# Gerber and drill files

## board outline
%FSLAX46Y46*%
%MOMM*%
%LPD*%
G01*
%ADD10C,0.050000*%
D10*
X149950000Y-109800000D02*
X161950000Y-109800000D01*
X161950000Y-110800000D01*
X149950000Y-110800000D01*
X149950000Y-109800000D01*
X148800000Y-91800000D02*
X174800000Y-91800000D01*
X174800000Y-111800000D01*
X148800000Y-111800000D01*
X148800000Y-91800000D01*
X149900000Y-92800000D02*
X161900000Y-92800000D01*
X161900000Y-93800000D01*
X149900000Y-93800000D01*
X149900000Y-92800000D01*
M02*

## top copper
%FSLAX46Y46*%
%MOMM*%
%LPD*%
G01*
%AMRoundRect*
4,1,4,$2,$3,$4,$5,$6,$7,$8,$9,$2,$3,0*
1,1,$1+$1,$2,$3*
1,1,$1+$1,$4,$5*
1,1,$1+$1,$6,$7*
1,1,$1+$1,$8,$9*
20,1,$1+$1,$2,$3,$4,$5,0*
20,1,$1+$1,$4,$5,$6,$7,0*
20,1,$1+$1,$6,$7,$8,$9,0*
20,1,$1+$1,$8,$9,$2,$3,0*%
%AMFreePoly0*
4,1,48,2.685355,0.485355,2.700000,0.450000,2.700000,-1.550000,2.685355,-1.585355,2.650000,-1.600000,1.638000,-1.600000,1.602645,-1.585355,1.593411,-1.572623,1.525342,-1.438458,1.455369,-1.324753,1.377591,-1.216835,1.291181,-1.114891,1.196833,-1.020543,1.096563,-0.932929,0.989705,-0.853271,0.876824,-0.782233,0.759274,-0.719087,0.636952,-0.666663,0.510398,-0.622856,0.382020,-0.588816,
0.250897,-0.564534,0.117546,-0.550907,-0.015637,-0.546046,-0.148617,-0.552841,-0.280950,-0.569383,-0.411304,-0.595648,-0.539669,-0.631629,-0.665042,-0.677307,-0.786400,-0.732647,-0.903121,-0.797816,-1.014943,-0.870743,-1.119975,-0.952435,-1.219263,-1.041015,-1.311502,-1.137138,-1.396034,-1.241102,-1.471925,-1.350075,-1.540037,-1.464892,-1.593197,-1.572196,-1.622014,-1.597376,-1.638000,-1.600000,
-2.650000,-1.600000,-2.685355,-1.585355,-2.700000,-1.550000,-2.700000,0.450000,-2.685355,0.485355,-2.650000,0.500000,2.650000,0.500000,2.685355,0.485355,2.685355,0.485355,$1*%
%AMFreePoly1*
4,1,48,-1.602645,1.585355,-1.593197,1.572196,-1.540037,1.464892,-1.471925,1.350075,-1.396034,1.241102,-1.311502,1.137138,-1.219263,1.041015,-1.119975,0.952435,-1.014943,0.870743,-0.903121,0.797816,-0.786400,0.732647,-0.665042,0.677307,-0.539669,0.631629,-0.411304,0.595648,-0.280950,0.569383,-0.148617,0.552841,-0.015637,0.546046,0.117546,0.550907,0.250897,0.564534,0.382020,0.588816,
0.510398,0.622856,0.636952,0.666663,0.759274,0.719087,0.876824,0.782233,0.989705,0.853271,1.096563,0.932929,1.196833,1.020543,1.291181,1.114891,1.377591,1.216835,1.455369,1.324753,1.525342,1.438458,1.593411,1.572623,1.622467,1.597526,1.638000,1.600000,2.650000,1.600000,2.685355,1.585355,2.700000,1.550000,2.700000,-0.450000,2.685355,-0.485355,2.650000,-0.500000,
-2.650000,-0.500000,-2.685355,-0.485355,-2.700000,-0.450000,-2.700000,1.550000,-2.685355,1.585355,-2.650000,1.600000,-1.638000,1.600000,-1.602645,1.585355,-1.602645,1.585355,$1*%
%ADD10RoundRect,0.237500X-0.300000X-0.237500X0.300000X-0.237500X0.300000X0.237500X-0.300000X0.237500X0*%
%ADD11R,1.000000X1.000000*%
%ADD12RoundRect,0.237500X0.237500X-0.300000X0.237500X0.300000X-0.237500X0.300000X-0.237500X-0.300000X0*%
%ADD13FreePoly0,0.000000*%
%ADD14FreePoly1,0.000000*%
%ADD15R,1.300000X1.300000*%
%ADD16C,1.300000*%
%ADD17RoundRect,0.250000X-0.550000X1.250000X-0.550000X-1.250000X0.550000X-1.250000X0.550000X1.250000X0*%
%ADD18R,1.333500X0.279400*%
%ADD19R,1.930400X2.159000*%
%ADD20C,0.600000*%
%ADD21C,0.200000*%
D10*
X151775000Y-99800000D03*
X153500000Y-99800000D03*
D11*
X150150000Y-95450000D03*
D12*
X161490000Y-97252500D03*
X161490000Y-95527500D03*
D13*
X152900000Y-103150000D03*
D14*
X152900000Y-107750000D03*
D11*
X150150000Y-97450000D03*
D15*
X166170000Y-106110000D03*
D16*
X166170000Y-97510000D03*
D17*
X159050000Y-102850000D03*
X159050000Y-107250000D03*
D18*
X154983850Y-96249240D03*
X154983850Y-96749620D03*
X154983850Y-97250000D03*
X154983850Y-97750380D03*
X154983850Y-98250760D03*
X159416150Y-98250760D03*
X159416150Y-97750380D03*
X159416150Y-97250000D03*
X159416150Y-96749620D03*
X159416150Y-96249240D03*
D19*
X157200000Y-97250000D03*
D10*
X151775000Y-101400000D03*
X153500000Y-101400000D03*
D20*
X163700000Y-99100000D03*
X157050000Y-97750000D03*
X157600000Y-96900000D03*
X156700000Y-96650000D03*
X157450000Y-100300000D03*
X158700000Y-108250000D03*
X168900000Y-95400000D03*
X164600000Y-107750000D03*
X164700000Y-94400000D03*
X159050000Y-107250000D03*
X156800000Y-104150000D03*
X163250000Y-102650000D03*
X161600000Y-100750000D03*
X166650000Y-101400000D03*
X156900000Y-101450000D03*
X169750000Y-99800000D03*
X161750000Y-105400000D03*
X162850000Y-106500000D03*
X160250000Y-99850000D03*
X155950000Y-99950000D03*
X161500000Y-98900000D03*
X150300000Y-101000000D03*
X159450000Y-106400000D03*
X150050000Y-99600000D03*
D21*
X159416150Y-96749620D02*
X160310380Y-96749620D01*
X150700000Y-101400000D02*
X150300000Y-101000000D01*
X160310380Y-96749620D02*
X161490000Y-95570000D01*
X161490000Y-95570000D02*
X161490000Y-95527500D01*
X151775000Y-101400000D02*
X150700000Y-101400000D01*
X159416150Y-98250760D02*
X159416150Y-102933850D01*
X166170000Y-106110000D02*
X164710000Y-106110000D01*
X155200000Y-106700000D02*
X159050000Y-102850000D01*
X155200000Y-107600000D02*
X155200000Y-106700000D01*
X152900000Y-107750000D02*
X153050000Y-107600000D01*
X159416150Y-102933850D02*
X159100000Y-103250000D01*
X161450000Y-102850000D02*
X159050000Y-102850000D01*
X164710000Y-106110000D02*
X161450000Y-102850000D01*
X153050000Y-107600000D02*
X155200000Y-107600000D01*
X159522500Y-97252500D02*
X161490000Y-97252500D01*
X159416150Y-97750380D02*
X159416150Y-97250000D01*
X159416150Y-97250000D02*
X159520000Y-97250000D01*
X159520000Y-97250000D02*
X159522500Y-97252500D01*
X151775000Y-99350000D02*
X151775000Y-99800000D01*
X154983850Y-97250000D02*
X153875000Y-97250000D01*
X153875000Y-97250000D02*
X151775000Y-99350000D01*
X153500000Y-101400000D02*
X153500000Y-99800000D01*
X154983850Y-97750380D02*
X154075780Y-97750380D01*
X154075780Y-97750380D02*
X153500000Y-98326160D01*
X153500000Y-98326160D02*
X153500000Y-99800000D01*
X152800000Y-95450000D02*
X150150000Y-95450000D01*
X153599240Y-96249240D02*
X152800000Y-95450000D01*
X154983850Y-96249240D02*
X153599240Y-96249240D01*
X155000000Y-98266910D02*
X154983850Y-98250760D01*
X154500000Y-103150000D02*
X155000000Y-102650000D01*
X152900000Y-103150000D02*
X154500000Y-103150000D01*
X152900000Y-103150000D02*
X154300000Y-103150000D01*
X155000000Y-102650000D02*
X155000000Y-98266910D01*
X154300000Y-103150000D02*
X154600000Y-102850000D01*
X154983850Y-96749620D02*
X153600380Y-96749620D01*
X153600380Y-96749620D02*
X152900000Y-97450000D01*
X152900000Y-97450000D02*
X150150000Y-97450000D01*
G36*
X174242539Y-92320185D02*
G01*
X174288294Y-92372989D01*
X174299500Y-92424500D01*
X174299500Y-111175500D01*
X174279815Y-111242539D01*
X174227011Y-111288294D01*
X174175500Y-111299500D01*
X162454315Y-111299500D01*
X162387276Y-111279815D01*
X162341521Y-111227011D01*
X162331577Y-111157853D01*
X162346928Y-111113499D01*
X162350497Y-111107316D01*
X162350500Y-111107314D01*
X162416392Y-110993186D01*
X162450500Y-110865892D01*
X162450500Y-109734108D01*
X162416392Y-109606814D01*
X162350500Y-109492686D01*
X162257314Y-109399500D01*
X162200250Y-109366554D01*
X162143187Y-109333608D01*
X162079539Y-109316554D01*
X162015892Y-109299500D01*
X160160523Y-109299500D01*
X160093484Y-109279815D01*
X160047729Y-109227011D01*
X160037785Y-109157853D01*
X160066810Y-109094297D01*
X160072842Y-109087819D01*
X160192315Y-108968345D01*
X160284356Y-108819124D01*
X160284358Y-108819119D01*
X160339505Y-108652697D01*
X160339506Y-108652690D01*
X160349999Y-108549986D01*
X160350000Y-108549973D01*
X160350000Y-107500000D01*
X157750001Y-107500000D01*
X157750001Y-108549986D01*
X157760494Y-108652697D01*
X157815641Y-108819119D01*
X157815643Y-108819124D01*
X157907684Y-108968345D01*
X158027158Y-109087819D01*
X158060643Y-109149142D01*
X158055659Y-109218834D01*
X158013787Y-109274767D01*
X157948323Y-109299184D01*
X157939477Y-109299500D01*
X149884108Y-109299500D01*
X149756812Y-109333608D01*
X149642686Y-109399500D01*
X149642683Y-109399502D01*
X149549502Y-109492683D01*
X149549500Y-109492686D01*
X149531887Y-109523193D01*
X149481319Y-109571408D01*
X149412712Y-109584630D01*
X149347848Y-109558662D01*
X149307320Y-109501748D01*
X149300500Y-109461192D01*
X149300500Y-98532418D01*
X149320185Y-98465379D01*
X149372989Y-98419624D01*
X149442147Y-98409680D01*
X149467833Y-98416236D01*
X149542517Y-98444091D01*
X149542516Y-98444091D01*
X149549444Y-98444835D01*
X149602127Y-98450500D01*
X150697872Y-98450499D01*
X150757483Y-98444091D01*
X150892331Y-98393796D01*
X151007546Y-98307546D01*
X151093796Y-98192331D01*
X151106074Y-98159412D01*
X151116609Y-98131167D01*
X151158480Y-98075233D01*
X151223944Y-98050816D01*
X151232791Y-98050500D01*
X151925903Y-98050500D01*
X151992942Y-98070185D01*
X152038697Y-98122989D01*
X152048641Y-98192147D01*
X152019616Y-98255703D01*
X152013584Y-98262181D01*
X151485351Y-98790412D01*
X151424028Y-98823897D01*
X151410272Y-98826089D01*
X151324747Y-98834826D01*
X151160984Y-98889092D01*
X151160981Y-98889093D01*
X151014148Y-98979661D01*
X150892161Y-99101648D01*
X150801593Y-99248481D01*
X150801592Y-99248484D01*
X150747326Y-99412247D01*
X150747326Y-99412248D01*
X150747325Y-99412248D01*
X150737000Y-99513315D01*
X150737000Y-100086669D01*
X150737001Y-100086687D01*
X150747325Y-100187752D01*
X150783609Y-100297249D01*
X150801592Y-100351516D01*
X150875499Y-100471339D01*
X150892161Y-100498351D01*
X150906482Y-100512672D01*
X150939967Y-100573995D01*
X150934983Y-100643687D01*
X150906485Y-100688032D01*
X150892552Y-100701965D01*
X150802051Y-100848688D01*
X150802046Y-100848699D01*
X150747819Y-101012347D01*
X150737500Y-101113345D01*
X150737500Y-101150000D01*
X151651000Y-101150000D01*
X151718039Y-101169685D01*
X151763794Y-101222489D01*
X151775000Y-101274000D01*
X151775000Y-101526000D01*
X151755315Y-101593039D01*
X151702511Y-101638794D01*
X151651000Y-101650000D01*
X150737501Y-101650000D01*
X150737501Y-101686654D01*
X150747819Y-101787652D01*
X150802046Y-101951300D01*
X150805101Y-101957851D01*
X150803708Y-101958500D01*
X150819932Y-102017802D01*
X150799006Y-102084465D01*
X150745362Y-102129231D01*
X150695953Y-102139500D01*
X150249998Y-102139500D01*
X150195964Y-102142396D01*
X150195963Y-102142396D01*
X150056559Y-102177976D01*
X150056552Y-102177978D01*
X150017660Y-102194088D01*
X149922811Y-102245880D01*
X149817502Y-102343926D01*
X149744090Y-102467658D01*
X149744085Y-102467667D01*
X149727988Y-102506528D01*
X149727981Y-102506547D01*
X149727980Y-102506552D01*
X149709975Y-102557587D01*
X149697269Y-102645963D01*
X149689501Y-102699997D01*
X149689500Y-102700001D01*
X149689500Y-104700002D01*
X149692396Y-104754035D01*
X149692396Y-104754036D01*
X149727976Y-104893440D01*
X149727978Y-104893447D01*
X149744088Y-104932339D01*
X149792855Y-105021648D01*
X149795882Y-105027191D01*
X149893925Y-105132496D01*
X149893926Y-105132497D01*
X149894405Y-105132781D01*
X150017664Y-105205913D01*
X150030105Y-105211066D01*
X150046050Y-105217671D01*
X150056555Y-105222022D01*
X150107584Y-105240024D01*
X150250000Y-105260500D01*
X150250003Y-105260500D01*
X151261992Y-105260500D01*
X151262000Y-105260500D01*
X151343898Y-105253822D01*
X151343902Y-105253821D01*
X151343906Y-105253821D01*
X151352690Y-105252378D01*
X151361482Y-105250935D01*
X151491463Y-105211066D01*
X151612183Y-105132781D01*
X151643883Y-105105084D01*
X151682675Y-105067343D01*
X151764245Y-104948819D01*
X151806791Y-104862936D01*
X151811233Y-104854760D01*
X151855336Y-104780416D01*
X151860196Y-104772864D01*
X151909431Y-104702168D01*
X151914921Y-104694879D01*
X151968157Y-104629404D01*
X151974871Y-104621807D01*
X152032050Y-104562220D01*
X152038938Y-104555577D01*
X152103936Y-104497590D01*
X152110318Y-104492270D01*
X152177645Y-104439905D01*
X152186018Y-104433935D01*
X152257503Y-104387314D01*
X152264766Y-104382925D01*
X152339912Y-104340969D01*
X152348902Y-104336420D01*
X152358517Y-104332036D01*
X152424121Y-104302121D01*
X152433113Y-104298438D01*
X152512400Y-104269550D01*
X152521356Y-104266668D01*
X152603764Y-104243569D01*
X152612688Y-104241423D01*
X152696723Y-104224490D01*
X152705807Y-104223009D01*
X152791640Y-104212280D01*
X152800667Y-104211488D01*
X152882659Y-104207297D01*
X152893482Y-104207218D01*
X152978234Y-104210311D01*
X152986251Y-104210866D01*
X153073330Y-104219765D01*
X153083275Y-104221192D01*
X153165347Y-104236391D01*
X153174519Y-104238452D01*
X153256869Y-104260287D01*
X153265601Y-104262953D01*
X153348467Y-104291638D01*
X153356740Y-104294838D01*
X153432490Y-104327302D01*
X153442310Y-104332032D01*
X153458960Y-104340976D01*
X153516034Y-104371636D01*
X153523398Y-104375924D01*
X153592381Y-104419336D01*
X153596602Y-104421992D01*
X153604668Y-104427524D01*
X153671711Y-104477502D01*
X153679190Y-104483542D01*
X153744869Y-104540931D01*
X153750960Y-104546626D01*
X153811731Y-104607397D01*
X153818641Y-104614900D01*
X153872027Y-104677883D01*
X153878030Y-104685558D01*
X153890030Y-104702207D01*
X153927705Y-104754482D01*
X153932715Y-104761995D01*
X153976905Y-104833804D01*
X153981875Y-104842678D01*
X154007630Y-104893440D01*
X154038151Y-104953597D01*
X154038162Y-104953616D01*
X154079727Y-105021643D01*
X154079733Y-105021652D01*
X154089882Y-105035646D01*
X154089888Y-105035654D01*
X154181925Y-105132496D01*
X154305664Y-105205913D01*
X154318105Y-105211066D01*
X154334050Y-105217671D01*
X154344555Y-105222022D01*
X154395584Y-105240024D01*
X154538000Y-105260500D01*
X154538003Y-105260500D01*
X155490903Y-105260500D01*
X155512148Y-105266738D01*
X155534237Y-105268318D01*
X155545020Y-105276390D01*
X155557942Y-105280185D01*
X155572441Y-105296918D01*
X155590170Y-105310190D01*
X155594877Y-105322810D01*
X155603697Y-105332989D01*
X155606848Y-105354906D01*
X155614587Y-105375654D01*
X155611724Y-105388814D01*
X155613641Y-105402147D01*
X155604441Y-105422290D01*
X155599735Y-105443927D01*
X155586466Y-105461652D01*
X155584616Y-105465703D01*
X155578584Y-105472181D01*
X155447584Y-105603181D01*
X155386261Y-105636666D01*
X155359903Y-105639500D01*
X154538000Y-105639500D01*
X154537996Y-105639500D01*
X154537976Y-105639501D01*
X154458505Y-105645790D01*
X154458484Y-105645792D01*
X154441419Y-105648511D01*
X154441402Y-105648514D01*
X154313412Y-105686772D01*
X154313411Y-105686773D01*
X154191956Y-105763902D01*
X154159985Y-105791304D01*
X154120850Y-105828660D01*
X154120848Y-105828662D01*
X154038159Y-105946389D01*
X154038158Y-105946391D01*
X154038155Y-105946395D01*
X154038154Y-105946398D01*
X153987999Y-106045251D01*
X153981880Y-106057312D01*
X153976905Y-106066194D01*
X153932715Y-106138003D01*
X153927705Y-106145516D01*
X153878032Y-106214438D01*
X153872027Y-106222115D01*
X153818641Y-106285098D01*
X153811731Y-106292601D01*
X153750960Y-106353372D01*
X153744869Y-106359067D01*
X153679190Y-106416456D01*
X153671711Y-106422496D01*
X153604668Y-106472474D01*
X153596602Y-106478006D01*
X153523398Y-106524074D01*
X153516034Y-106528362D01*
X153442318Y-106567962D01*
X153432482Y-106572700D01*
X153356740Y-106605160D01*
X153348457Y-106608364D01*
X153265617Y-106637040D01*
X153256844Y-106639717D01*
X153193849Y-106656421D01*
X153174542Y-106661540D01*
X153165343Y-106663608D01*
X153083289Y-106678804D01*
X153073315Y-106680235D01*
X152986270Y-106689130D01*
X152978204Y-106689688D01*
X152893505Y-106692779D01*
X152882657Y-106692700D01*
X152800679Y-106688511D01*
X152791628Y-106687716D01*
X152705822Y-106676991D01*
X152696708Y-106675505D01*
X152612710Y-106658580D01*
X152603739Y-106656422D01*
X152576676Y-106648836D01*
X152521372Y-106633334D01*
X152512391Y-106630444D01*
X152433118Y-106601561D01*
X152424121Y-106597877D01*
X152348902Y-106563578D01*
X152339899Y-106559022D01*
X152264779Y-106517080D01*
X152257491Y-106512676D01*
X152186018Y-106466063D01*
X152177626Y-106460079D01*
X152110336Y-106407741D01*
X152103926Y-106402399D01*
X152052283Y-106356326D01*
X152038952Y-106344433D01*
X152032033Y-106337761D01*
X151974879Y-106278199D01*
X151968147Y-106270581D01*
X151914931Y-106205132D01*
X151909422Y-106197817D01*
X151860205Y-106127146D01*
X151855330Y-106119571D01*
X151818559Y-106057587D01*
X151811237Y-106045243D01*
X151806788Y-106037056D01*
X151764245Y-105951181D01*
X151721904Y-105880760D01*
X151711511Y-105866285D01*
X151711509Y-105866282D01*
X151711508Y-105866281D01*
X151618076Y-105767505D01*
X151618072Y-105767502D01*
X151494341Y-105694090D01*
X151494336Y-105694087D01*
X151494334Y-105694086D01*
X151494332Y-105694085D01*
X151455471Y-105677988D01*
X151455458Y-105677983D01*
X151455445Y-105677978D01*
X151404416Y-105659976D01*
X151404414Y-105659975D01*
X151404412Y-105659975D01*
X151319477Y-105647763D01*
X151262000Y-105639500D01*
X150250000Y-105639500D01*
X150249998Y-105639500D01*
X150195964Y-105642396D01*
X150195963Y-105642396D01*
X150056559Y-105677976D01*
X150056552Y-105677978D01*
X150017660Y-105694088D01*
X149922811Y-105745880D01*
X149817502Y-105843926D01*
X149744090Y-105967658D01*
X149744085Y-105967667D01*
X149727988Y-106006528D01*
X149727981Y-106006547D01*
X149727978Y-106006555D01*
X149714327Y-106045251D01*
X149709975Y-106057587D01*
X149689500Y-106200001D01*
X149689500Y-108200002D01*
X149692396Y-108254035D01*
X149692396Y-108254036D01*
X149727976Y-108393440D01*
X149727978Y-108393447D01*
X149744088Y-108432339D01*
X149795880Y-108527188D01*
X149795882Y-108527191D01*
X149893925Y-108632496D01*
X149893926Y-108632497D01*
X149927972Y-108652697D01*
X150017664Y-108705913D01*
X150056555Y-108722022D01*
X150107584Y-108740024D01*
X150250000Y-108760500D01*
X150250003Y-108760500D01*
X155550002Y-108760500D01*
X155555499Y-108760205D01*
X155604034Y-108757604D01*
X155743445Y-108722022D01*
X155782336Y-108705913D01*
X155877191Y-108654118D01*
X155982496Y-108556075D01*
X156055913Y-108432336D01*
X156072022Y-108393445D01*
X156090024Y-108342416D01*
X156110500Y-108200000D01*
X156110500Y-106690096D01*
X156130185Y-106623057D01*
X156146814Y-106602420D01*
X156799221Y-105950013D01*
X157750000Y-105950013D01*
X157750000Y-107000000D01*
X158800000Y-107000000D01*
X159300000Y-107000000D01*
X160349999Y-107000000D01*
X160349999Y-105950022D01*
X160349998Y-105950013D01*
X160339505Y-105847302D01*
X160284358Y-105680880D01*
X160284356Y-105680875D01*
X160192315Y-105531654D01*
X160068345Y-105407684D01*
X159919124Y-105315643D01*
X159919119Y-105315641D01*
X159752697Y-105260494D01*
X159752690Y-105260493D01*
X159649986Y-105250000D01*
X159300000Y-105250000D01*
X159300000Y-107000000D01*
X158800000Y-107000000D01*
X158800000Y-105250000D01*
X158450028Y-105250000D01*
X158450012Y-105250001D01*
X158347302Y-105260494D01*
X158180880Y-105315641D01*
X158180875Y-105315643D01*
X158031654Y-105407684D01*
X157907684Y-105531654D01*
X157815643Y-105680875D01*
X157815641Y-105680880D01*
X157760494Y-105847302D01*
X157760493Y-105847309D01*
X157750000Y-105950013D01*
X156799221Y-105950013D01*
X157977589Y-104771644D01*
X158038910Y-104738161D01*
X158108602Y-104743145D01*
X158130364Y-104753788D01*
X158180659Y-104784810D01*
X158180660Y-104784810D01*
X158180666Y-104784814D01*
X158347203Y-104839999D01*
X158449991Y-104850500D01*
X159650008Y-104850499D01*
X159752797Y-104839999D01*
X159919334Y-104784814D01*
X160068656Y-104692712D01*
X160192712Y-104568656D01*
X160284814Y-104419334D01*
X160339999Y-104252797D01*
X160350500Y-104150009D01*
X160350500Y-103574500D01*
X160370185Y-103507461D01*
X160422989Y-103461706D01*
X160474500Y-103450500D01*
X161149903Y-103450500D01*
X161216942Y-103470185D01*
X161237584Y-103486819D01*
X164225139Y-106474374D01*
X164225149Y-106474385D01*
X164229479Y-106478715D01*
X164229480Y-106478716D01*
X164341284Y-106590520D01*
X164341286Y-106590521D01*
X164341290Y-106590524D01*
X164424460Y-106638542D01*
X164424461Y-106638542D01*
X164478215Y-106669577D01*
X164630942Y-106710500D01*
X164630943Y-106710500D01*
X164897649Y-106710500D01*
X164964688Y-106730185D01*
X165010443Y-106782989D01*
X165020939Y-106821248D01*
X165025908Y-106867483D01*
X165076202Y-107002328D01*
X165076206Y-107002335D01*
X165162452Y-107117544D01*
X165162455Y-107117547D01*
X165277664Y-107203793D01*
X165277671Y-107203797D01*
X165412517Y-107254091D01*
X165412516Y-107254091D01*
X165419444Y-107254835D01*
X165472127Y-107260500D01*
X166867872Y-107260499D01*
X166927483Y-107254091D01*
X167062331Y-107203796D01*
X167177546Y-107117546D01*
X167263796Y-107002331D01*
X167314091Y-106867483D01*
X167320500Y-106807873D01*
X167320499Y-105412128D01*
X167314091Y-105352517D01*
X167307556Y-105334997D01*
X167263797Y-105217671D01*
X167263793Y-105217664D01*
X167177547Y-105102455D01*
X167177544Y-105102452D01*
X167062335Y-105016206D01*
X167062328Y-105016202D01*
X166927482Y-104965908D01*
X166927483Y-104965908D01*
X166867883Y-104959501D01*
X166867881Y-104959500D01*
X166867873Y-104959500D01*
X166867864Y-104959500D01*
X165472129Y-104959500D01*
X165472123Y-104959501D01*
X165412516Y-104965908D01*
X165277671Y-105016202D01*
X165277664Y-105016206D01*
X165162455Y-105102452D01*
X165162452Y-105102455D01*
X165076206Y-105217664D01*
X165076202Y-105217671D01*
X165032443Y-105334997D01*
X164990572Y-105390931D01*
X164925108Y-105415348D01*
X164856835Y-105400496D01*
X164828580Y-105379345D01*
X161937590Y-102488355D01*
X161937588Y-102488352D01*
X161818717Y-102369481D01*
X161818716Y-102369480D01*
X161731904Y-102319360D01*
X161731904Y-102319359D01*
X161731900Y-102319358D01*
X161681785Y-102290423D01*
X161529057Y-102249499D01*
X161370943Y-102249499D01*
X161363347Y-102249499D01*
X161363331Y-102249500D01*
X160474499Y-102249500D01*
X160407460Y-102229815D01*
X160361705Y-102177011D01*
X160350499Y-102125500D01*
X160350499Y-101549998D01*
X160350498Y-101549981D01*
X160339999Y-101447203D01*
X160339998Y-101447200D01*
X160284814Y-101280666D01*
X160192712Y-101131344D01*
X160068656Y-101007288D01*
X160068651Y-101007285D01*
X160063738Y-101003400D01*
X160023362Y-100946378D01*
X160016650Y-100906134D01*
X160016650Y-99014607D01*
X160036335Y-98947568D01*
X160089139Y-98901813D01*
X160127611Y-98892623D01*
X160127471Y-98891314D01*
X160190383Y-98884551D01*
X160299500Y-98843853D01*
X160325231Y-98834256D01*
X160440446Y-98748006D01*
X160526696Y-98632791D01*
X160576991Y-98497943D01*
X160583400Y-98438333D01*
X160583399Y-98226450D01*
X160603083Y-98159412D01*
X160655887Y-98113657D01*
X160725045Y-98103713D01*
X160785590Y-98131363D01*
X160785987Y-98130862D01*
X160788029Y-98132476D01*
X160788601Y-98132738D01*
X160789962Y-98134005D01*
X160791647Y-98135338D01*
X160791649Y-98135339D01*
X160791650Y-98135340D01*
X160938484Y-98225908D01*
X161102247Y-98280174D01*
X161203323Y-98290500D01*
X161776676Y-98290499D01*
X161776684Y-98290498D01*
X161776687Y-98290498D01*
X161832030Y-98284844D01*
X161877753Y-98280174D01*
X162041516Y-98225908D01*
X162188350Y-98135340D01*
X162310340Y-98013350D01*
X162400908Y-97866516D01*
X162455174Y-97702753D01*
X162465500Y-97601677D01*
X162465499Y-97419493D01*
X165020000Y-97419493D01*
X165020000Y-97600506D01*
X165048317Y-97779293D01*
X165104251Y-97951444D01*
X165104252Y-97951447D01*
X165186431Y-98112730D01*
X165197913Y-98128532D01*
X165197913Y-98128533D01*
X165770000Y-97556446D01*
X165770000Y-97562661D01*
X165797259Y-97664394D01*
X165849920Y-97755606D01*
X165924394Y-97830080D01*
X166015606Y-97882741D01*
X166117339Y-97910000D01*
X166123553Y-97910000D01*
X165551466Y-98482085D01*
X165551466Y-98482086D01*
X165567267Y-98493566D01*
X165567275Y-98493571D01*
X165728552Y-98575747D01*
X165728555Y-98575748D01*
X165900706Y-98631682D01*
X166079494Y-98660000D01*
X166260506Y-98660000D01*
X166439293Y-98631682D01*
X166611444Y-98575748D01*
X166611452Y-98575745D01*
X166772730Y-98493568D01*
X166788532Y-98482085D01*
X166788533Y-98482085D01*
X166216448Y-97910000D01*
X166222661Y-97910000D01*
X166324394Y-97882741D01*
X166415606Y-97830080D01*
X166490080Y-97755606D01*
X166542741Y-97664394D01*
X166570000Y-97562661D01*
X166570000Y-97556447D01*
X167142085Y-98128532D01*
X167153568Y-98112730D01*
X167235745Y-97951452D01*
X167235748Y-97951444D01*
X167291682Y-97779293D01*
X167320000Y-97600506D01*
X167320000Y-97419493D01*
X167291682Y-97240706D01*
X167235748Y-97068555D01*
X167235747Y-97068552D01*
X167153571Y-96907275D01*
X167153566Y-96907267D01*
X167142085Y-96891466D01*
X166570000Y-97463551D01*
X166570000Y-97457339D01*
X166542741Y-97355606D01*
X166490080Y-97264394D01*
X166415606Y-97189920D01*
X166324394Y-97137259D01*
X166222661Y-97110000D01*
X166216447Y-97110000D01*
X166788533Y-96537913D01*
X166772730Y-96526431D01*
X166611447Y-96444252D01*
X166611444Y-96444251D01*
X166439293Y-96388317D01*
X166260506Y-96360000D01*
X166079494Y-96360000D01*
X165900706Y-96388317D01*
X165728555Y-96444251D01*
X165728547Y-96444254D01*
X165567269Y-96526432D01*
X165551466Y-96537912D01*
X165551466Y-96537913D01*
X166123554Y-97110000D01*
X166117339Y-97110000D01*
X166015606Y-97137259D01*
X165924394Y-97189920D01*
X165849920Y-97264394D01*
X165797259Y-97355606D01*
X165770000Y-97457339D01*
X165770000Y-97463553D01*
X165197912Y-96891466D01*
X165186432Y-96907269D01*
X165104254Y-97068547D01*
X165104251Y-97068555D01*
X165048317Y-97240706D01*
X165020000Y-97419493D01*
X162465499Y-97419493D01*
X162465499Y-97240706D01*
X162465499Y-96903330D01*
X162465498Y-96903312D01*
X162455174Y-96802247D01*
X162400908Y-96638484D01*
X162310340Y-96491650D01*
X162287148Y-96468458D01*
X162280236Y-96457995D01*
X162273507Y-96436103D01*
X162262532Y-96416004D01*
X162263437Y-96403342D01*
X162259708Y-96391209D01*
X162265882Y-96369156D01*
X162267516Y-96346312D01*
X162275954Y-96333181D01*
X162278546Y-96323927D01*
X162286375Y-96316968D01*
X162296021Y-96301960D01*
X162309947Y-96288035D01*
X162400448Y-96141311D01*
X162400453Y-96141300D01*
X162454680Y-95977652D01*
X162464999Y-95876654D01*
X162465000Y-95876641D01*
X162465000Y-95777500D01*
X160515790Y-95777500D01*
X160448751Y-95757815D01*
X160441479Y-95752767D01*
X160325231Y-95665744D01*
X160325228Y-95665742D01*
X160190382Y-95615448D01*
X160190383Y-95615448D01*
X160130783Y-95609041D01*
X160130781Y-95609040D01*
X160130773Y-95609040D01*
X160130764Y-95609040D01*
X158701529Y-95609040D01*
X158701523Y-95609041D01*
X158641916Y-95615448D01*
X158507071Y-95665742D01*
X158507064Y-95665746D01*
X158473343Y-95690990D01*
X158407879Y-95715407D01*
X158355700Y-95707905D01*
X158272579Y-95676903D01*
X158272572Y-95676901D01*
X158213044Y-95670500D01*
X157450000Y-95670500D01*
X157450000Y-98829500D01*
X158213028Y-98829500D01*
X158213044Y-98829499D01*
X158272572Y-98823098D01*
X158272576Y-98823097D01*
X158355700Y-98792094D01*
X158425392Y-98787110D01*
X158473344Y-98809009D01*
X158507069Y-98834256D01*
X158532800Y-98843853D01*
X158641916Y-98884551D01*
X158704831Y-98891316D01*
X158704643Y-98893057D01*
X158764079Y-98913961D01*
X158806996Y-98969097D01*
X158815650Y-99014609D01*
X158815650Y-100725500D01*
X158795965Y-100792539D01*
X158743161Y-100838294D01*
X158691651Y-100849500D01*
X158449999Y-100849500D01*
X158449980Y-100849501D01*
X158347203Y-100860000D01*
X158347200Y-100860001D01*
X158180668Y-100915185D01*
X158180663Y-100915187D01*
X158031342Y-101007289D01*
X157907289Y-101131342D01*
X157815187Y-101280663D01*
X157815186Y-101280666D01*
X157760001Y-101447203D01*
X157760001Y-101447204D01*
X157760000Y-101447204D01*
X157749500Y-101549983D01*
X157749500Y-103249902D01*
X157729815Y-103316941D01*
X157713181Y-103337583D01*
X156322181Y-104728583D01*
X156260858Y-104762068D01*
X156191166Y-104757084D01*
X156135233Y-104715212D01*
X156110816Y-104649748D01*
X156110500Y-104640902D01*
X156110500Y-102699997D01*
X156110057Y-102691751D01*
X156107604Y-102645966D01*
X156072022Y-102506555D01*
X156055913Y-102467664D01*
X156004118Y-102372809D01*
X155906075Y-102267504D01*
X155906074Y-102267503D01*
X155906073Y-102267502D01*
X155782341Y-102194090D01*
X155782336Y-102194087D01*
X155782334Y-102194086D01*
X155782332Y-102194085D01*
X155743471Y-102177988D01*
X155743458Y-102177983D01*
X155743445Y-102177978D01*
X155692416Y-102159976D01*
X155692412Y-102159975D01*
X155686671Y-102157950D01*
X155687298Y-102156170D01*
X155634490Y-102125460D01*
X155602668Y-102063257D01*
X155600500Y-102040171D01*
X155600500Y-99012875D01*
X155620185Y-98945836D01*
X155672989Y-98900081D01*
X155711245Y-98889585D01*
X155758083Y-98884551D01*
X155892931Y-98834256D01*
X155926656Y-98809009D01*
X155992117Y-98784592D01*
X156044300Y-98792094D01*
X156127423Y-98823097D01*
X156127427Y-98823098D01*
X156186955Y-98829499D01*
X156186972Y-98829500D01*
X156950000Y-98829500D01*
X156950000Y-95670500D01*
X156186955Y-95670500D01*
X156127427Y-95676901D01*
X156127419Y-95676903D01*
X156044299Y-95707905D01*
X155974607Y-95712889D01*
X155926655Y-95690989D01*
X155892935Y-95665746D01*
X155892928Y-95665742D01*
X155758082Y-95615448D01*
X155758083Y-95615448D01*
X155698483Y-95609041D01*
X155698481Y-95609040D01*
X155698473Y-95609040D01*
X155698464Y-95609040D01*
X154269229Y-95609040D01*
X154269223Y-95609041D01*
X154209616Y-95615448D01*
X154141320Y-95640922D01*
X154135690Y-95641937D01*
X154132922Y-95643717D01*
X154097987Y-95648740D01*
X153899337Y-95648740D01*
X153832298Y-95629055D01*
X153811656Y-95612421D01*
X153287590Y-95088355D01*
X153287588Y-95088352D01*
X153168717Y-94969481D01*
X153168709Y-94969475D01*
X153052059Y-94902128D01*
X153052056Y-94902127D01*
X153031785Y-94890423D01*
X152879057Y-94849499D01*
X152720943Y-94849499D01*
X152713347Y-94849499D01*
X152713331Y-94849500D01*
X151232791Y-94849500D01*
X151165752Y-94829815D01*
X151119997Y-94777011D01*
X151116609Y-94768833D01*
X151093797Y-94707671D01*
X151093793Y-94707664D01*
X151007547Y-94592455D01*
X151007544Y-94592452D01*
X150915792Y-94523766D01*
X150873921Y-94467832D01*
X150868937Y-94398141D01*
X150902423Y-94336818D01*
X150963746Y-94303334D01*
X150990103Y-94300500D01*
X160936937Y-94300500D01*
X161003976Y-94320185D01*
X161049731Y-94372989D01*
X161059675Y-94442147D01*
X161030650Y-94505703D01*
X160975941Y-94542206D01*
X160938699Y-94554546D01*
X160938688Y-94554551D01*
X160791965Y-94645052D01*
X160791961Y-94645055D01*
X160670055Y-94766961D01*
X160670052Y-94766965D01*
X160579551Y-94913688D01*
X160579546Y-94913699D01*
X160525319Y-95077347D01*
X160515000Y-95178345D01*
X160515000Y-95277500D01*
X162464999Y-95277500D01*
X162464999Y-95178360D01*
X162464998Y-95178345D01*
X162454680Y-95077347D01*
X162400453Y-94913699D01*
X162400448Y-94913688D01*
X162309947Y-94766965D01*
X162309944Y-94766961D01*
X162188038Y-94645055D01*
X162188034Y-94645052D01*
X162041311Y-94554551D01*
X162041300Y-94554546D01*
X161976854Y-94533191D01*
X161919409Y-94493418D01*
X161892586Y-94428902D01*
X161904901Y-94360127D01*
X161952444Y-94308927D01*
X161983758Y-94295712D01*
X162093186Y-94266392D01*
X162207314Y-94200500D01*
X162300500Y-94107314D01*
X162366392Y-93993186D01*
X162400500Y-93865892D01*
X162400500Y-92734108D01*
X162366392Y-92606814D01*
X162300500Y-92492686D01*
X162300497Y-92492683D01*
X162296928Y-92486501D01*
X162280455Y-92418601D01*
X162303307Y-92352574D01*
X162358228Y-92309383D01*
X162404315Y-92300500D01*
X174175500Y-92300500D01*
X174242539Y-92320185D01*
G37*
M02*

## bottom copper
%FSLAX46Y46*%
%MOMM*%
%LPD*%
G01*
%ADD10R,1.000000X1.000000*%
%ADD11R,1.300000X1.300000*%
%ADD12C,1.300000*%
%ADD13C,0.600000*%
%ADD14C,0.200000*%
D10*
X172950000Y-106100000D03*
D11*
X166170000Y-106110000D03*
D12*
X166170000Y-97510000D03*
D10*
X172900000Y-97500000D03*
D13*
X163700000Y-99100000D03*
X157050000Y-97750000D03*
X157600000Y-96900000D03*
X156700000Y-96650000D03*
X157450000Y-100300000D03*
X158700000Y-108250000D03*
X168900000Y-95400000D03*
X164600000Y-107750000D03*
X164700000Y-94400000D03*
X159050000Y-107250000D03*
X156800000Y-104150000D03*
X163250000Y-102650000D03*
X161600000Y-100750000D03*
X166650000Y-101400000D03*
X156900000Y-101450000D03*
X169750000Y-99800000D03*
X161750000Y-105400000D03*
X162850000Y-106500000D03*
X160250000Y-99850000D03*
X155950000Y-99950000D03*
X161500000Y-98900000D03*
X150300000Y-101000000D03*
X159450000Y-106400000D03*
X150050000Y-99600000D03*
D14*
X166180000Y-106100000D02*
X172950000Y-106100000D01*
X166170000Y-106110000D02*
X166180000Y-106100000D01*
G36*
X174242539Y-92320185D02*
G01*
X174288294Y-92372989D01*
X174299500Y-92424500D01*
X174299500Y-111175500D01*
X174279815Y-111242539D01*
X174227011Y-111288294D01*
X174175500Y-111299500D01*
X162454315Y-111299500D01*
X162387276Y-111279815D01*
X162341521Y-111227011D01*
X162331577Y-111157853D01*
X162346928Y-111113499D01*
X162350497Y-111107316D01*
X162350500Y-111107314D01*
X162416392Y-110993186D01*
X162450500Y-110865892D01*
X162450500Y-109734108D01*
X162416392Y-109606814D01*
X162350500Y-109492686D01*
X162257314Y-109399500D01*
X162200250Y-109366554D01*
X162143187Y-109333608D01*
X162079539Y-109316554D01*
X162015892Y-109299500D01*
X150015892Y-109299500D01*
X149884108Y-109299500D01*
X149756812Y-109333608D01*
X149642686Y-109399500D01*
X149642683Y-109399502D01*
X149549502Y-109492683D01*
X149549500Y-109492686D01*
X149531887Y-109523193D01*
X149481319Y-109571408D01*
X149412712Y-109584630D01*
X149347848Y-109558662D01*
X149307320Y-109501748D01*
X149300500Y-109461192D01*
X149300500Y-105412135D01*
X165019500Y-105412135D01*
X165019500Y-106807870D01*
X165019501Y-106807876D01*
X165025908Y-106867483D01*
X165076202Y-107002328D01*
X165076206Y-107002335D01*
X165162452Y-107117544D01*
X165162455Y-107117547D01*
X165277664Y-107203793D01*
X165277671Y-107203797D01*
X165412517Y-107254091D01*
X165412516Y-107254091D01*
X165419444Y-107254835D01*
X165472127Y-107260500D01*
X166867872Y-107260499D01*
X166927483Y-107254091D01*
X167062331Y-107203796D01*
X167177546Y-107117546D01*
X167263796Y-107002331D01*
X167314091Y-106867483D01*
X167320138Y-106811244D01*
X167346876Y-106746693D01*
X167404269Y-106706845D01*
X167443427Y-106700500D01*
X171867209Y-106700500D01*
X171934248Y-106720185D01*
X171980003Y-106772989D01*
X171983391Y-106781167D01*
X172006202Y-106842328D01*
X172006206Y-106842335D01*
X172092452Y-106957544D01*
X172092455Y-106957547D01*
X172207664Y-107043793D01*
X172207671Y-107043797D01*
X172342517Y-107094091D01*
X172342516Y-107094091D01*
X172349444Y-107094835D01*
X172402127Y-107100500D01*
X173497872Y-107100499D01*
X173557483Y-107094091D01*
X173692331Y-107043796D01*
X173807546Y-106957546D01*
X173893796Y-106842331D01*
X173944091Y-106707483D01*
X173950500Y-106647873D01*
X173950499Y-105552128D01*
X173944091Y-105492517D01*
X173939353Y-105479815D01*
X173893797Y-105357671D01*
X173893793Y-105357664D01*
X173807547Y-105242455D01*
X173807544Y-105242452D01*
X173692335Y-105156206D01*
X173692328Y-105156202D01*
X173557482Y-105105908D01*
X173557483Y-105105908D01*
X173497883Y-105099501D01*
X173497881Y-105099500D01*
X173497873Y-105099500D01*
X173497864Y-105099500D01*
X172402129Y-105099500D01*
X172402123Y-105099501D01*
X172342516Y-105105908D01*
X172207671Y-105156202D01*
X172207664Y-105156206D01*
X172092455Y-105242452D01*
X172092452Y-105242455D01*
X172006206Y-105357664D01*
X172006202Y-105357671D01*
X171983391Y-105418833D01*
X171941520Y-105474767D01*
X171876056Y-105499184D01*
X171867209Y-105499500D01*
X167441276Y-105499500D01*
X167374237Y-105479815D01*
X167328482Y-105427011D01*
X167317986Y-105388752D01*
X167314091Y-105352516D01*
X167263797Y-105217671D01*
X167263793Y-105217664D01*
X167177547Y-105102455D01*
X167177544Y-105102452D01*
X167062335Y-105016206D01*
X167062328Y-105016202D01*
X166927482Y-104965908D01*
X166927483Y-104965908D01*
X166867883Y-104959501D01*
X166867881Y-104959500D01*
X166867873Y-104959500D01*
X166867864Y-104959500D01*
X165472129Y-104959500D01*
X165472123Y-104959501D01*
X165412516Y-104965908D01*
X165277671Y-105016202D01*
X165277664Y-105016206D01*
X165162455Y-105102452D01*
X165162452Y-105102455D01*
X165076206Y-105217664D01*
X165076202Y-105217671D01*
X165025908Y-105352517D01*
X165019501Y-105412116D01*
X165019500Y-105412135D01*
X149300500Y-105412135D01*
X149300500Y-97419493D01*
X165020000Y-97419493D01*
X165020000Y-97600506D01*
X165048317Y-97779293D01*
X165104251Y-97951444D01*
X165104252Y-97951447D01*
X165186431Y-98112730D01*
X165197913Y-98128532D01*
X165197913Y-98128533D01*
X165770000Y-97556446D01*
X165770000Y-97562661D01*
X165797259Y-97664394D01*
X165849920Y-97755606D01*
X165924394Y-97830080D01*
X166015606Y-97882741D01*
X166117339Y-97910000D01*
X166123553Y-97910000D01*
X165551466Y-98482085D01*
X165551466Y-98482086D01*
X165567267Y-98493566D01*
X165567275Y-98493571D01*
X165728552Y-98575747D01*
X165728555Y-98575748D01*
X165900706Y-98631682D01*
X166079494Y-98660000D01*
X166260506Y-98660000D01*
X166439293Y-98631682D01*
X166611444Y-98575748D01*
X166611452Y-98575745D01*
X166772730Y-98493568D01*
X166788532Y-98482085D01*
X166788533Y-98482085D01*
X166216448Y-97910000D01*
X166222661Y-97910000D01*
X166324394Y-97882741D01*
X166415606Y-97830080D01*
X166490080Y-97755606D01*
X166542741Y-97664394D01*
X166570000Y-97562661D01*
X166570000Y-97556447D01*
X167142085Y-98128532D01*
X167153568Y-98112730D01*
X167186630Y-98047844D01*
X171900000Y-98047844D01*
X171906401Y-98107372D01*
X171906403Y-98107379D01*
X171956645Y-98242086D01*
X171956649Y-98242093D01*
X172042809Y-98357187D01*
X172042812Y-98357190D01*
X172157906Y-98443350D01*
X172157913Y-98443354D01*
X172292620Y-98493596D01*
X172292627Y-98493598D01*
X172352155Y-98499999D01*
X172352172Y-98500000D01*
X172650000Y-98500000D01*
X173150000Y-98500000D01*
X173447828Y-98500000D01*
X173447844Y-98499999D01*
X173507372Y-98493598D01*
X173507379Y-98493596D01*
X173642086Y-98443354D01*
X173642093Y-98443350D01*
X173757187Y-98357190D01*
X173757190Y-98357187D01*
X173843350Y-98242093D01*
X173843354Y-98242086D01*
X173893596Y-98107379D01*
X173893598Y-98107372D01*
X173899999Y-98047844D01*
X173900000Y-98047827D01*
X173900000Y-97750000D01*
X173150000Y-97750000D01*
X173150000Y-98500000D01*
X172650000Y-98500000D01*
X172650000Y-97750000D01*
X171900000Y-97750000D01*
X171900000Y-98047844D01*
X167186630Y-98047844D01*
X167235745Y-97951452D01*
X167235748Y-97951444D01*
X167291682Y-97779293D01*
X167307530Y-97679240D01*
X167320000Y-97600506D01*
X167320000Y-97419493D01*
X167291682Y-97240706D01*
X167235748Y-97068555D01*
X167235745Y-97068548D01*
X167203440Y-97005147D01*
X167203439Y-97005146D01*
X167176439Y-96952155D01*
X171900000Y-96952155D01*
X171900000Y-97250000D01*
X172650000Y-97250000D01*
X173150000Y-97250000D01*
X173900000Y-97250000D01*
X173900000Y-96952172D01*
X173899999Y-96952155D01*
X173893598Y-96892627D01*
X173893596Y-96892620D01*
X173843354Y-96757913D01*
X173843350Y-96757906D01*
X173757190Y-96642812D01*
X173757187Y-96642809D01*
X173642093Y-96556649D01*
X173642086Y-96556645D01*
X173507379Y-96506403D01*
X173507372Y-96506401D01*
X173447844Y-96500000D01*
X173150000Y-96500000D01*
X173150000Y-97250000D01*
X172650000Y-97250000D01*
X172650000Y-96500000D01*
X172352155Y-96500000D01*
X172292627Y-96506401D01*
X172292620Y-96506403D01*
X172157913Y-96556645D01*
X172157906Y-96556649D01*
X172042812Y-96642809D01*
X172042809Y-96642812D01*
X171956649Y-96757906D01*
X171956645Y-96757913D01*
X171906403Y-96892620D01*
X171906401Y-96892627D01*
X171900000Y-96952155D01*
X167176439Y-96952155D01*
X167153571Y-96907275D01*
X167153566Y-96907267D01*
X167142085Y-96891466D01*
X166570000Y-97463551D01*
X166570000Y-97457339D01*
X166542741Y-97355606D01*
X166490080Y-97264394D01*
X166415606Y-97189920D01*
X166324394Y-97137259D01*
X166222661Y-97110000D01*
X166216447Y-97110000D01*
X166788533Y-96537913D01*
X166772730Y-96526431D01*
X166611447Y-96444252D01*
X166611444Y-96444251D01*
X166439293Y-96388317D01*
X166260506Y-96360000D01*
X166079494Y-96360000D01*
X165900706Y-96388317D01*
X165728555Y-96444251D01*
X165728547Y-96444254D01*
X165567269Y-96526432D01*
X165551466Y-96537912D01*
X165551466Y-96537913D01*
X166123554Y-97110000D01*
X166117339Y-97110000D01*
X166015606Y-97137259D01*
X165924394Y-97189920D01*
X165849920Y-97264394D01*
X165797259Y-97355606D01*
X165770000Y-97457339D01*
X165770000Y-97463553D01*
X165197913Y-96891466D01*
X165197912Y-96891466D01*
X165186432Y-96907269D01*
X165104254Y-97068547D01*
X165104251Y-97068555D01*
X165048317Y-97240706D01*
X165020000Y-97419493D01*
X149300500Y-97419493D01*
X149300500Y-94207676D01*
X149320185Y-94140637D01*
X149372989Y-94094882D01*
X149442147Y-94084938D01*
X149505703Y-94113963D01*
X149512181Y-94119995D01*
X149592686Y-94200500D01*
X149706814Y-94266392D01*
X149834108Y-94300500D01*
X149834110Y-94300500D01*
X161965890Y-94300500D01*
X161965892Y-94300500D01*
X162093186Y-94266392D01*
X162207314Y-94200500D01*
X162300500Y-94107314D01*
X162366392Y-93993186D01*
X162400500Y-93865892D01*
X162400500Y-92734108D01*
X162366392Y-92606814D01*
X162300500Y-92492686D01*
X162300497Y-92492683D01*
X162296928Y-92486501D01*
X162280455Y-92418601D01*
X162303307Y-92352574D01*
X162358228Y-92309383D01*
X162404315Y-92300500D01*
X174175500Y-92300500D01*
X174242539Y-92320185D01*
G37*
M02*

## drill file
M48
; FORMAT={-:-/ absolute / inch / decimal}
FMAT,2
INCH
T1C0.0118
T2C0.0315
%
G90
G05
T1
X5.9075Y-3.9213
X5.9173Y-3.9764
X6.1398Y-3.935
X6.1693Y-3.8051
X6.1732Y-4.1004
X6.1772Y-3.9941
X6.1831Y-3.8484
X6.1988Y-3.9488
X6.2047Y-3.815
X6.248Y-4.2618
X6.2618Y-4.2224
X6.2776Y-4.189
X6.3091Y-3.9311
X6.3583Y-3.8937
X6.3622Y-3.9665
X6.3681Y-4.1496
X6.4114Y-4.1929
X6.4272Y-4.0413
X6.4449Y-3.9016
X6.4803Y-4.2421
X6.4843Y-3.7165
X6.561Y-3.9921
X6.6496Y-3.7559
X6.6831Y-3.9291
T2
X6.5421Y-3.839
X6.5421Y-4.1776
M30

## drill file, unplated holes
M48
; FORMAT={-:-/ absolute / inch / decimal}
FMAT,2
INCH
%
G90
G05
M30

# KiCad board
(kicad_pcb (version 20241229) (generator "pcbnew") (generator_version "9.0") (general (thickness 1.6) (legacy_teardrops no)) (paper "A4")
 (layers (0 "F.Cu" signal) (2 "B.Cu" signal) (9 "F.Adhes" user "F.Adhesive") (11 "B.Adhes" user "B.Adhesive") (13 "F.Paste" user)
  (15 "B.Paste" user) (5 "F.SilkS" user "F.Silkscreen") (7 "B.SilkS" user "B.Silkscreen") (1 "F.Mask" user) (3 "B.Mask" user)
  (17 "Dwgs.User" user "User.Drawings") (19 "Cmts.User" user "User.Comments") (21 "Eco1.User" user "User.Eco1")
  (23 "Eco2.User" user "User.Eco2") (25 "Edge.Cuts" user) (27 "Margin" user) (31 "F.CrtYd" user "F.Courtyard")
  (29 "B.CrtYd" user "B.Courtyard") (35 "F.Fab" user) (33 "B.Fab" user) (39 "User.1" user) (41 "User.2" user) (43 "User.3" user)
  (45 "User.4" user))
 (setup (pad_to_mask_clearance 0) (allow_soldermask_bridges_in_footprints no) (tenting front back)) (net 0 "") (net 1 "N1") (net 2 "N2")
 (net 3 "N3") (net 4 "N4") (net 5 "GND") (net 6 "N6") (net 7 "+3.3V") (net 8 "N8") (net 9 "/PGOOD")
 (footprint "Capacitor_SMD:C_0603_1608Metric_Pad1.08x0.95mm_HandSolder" (layer "F.Cu") (at 152.6375 99.8)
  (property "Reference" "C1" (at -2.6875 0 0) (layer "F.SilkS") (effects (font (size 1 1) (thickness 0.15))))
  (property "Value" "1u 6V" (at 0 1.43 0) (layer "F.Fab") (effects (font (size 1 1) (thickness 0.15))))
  (pad "1" smd roundrect (at -0.8625 0) (size 1.075 0.95) (layers "F.Cu" "F.Mask" "F.Paste") (roundrect_rratio 0.25) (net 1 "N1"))
  (pad "2" smd roundrect (at 0.8625 0) (size 1.075 0.95) (layers "F.Cu" "F.Mask" "F.Paste") (roundrect_rratio 0.25) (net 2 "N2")))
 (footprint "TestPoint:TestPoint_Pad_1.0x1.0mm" (layer "F.Cu") (at 150.15 95.45)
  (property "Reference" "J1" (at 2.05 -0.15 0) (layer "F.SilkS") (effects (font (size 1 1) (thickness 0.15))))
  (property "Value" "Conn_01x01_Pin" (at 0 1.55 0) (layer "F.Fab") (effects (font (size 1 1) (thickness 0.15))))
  (pad "1" smd rect (at 0 0) (size 1 1) (layers "F.Cu" "F.Mask") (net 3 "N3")))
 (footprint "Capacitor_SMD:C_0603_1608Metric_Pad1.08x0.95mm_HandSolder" (layer "F.Cu") (at 161.49 96.39 90)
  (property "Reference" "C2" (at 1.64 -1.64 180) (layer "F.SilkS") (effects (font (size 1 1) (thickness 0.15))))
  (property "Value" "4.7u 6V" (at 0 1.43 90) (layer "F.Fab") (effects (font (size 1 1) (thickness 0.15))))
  (pad "1" smd roundrect (at -0.8625 0 90) (size 1.075 0.95) (layers "F.Cu" "F.Mask" "F.Paste") (roundrect_rratio 0.25) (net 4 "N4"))
  (pad "2" smd roundrect (at 0.8625 0 90) (size 1.075 0.95) (layers "F.Cu" "F.Mask" "F.Paste") (roundrect_rratio 0.25) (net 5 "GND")))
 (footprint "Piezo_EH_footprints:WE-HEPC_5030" (layer "F.Cu") (at 152.9 105.45)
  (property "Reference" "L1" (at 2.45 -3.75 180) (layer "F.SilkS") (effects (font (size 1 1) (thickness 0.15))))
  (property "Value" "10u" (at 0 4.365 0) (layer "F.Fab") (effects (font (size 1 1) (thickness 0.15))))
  (pad "1" smd custom (at 0 -2.3) (size 5.3 0.9) (layers "F.Cu") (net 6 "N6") (options (clearance outline) (anchor rect)) (primitives))
  (pad "2" smd custom (at 0 2.3) (size 5.1 0.9) (layers "F.Cu") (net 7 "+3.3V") (options (clearance outline) (anchor rect)) (primitives)))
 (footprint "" (layer "F.Cu") (at 172.95 106.1)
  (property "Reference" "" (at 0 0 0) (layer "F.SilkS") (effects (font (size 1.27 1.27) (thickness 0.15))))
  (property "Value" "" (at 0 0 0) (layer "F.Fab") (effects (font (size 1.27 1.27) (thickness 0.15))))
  (pad "3" smd rect (at 0 0) (size 1 1) (layers "B.Cu" "B.Mask") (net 7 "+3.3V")))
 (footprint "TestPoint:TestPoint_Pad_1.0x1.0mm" (layer "F.Cu") (at 150.15 97.45)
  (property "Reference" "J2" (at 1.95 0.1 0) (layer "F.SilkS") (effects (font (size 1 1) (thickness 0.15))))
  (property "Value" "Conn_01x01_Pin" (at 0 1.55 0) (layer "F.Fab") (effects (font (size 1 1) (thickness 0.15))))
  (pad "1" smd rect (at 0 0) (size 1 1) (layers "F.Cu" "F.Mask") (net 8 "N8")))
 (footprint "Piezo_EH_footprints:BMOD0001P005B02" (layer "F.Cu") (at 166.17 106.11 90)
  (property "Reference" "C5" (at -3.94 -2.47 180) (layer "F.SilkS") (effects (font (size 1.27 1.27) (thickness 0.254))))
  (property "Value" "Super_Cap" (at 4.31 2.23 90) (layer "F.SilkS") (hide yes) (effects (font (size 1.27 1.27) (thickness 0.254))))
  (pad "1" thru_hole rect (at 0 0 90) (size 1.3 1.3) (drill 0.8) (layers "*.Cu" "*.Mask") (remove_unused_layers no) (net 7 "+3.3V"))
  (pad "2" thru_hole circle (at 8.6 0 90) (size 1.3 1.3) (drill 0.8) (layers "*.Cu" "*.Mask") (remove_unused_layers no) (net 5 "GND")))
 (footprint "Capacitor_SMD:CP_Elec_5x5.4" (layer "F.Cu") (at 159.05 105.05 -90)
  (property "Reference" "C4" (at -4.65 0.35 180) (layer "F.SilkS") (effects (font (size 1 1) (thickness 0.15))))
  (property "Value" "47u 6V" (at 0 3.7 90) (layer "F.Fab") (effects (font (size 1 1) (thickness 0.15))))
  (pad "1" smd roundrect (at -2.2 0 270) (size 3 1.6) (layers "F.Cu" "F.Mask" "F.Paste") (roundrect_rratio 0.15625) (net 7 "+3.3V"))
  (pad "2" smd roundrect (at 2.2 0 270) (size 3 1.6) (layers "F.Cu" "F.Mask" "F.Paste") (roundrect_rratio 0.15625) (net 5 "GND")))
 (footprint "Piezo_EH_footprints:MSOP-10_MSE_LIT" (layer "F.Cu") (at 157.2 97.25)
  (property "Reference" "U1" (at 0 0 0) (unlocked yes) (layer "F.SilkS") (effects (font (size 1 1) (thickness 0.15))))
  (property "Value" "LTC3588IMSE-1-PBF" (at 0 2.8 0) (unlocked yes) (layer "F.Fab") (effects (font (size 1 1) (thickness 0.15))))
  (pad "1" smd rect (at -2.21615 -1.00076) (size 1.3335 0.2794) (layers "F.Cu" "F.Mask" "F.Paste") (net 3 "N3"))
  (pad "2" smd rect (at -2.21615 -0.50038) (size 1.3335 0.2794) (layers "F.Cu" "F.Mask" "F.Paste") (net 8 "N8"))
  (pad "3" smd rect (at -2.21615 0) (size 1.3335 0.2794) (layers "F.Cu" "F.Mask" "F.Paste") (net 1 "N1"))
  (pad "4" smd rect (at -2.21615 0.50038) (size 1.3335 0.2794) (layers "F.Cu" "F.Mask" "F.Paste") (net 2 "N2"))
  (pad "5" smd rect (at -2.21615 1.00076) (size 1.3335 0.2794) (layers "F.Cu" "F.Mask" "F.Paste") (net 6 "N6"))
  (pad "6" smd rect (at 2.21615 1.00076) (size 1.3335 0.2794) (layers "F.Cu" "F.Mask" "F.Paste") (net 7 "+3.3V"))
  (pad "7" smd rect (at 2.21615 0.50038) (size 1.3335 0.2794) (layers "F.Cu" "F.Mask" "F.Paste") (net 4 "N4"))
  (pad "8" smd rect (at 2.21615 0) (size 1.3335 0.2794) (layers "F.Cu" "F.Mask" "F.Paste") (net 4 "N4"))
  (pad "9" smd rect (at 2.21615 -0.50038) (size 1.3335 0.2794) (layers "F.Cu" "F.Mask" "F.Paste") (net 5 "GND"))
  (pad "10" smd rect (at 2.21615 -1.00076) (size 1.3335 0.2794) (layers "F.Cu" "F.Mask" "F.Paste") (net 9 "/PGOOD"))
  (pad "EPAD" smd rect (at 0 0) (size 1.9304 2.159) (layers "F.Cu" "F.Mask" "F.Paste") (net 5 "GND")))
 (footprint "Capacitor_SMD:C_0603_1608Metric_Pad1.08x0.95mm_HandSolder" (layer "F.Cu") (at 152.6375 101.4)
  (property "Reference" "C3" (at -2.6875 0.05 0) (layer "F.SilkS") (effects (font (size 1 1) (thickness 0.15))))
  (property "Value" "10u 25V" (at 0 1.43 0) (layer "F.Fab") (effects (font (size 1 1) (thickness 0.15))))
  (pad "1" smd roundrect (at -0.8625 0) (size 1.075 0.95) (layers "F.Cu" "F.Mask" "F.Paste") (roundrect_rratio 0.25) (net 5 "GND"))
  (pad "2" smd roundrect (at 0.8625 0) (size 1.075 0.95) (layers "F.Cu" "F.Mask" "F.Paste") (roundrect_rratio 0.25) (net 2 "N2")))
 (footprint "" (layer "F.Cu") (at 172.9 97.5)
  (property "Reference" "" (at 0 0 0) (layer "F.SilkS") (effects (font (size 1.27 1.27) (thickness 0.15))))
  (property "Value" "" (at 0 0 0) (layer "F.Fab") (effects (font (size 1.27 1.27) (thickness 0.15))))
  (pad "4" smd rect (at 0 0) (size 1 1) (layers "B.Cu" "B.Mask") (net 5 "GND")))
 (gr_rect (start 149.95 109.8) (end 161.95 110.8) (stroke (width 0.05) (type default)) (fill no) (layer "Edge.Cuts"))
 (gr_rect (start 148.8 91.8) (end 174.8 111.8) (stroke (width 0.05) (type default)) (fill no) (layer "Edge.Cuts"))
 (gr_rect (start 149.9 92.8) (end 161.9 93.8) (stroke (width 0.05) (type default)) (fill no) (layer "Edge.Cuts"))
 (segment (start 159.41615 96.74962) (end 160.31038 96.74962) (width 0.2) (layer "F.Cu") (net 5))
 (segment (start 150.7 101.4) (end 150.3 101) (width 0.2) (layer "F.Cu") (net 5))
 (segment (start 160.31038 96.74962) (end 161.49 95.57) (width 0.2) (layer "F.Cu") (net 5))
 (segment (start 161.49 95.57) (end 161.49 95.5275) (width 0.2) (layer "F.Cu") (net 5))
 (segment (start 151.775 101.4) (end 150.7 101.4) (width 0.2) (layer "F.Cu") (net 5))
 (via (at 163.7 99.1) (size 0.6) (drill 0.3) (layers "F.Cu" "B.Cu") (free yes) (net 5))
 (via (at 157.05 97.75) (size 0.6) (drill 0.3) (layers "F.Cu" "B.Cu") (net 5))
 (via (at 157.6 96.9) (size 0.6) (drill 0.3) (layers "F.Cu" "B.Cu") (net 5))
 (via (at 156.7 96.65) (size 0.6) (drill 0.3) (layers "F.Cu" "B.Cu") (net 5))
 (via (at 157.45 100.3) (size 0.6) (drill 0.3) (layers "F.Cu" "B.Cu") (free yes) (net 5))
 (via (at 158.7 108.25) (size 0.6) (drill 0.3) (layers "F.Cu" "B.Cu") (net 5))
 (via (at 168.9 95.4) (size 0.6) (drill 0.3) (layers "F.Cu" "B.Cu") (free yes) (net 5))
 (via (at 164.6 107.75) (size 0.6) (drill 0.3) (layers "F.Cu" "B.Cu") (free yes) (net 5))
 (via (at 164.7 94.4) (size 0.6) (drill 0.3) (layers "F.Cu" "B.Cu") (free yes) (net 5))
 (via (at 159.05 107.25) (size 0.6) (drill 0.3) (layers "F.Cu" "B.Cu") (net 5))
 (via (at 156.8 104.15) (size 0.6) (drill 0.3) (layers "F.Cu" "B.Cu") (free yes) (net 5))
 (via (at 163.25 102.65) (size 0.6) (drill 0.3) (layers "F.Cu" "B.Cu") (free yes) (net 5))
 (via (at 161.6 100.75) (size 0.6) (drill 0.3) (layers "F.Cu" "B.Cu") (free yes) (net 5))
 (via (at 166.65 101.4) (size 0.6) (drill 0.3) (layers "F.Cu" "B.Cu") (free yes) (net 5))
 (via (at 156.9 101.45) (size 0.6) (drill 0.3) (layers "F.Cu" "B.Cu") (free yes) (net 5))
 (via (at 169.75 99.8) (size 0.6) (drill 0.3) (layers "F.Cu" "B.Cu") (free yes) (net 5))
 (via (at 161.75 105.4) (size 0.6) (drill 0.3) (layers "F.Cu" "B.Cu") (free yes) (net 5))
 (via (at 162.85 106.5) (size 0.6) (drill 0.3) (layers "F.Cu" "B.Cu") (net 5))
 (via (at 160.25 99.85) (size 0.6) (drill 0.3) (layers "F.Cu" "B.Cu") (free yes) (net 5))
 (via (at 155.95 99.95) (size 0.6) (drill 0.3) (layers "F.Cu" "B.Cu") (free yes) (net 5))
 (via (at 161.5 98.9) (size 0.6) (drill 0.3) (layers "F.Cu" "B.Cu") (free yes) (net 5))
 (via (at 150.3 101) (size 0.6) (drill 0.3) (layers "F.Cu" "B.Cu") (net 5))
 (via (at 159.45 106.4) (size 0.6) (drill 0.3) (layers "F.Cu" "B.Cu") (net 5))
 (via (at 150.05 99.6) (size 0.6) (drill 0.3) (layers "F.Cu" "B.Cu") (free yes) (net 5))
 (segment (start 159.41615 98.25076) (end 159.41615 102.93385) (width 0.2) (layer "F.Cu") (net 7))
 (segment (start 166.17 106.11) (end 164.71 106.11) (width 0.2) (layer "F.Cu") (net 7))
 (segment (start 155.2 106.7) (end 159.05 102.85) (width 0.2) (layer "F.Cu") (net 7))
 (segment (start 155.2 107.6) (end 155.2 106.7) (width 0.2) (layer "F.Cu") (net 7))
 (segment (start 152.9 107.75) (end 153.05 107.6) (width 0.2) (layer "F.Cu") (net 7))
 (segment (start 159.41615 102.93385) (end 159.1 103.25) (width 0.2) (layer "F.Cu") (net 7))
 (segment (start 161.45 102.85) (end 159.05 102.85) (width 0.2) (layer "F.Cu") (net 7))
 (segment (start 164.71 106.11) (end 161.45 102.85) (width 0.2) (layer "F.Cu") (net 7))
 (segment (start 153.05 107.6) (end 155.2 107.6) (width 0.2) (layer "F.Cu") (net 7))
 (segment (start 166.18 106.1) (end 172.95 106.1) (width 0.2) (layer "B.Cu") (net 7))
 (segment (start 166.17 106.11) (end 166.18 106.1) (width 0.2) (layer "B.Cu") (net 7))
 (segment (start 159.5225 97.2525) (end 161.49 97.2525) (width 0.2) (layer "F.Cu") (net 4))
 (segment (start 159.41615 97.75038) (end 159.41615 97.25) (width 0.2) (layer "F.Cu") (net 4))
 (segment (start 159.41615 97.25) (end 159.52 97.25) (width 0.2) (layer "F.Cu") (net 4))
 (segment (start 159.52 97.25) (end 159.5225 97.2525) (width 0.2) (layer "F.Cu") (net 4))
 (segment (start 151.775 99.35) (end 151.775 99.8) (width 0.2) (layer "F.Cu") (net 1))
 (segment (start 154.98385 97.25) (end 153.875 97.25) (width 0.2) (layer "F.Cu") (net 1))
 (segment (start 153.875 97.25) (end 151.775 99.35) (width 0.2) (layer "F.Cu") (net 1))
 (segment (start 153.5 101.4) (end 153.5 99.8) (width 0.2) (layer "F.Cu") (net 2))
 (segment (start 154.98385 97.75038) (end 154.07578 97.75038) (width 0.2) (layer "F.Cu") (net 2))
 (segment (start 154.07578 97.75038) (end 153.5 98.32616) (width 0.2) (layer "F.Cu") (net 2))
 (segment (start 153.5 98.32616) (end 153.5 99.8) (width 0.2) (layer "F.Cu") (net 2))
 (segment (start 152.8 95.45) (end 150.15 95.45) (width 0.2) (layer "F.Cu") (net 3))
 (segment (start 153.59924 96.24924) (end 152.8 95.45) (width 0.2) (layer "F.Cu") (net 3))
 (segment (start 154.98385 96.24924) (end 153.59924 96.24924) (width 0.2) (layer "F.Cu") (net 3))
 (segment (start 155 98.26691) (end 154.98385 98.25076) (width 0.2) (layer "F.Cu") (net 6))
 (segment (start 154.5 103.15) (end 155 102.65) (width 0.2) (layer "F.Cu") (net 6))
 (segment (start 152.9 103.15) (end 154.5 103.15) (width 0.2) (layer "F.Cu") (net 6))
 (segment (start 152.9 103.15) (end 154.3 103.15) (width 0.2) (layer "F.Cu") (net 6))
 (segment (start 155 102.65) (end 155 98.26691) (width 0.2) (layer "F.Cu") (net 6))
 (segment (start 154.3 103.15) (end 154.6 102.85) (width 0.2) (layer "F.Cu") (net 6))
 (segment (start 154.98385 96.74962) (end 153.60038 96.74962) (width 0.2) (layer "F.Cu") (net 8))
 (segment (start 153.60038 96.74962) (end 152.9 97.45) (width 0.2) (layer "F.Cu") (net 8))
 (segment (start 152.9 97.45) (end 150.15 97.45) (width 0.2) (layer "F.Cu") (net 8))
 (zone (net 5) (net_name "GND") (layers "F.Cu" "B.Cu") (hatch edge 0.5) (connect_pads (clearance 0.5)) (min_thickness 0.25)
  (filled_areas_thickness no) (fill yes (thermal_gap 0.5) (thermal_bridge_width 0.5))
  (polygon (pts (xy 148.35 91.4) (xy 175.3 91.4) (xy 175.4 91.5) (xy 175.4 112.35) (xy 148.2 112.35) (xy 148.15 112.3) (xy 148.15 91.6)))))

